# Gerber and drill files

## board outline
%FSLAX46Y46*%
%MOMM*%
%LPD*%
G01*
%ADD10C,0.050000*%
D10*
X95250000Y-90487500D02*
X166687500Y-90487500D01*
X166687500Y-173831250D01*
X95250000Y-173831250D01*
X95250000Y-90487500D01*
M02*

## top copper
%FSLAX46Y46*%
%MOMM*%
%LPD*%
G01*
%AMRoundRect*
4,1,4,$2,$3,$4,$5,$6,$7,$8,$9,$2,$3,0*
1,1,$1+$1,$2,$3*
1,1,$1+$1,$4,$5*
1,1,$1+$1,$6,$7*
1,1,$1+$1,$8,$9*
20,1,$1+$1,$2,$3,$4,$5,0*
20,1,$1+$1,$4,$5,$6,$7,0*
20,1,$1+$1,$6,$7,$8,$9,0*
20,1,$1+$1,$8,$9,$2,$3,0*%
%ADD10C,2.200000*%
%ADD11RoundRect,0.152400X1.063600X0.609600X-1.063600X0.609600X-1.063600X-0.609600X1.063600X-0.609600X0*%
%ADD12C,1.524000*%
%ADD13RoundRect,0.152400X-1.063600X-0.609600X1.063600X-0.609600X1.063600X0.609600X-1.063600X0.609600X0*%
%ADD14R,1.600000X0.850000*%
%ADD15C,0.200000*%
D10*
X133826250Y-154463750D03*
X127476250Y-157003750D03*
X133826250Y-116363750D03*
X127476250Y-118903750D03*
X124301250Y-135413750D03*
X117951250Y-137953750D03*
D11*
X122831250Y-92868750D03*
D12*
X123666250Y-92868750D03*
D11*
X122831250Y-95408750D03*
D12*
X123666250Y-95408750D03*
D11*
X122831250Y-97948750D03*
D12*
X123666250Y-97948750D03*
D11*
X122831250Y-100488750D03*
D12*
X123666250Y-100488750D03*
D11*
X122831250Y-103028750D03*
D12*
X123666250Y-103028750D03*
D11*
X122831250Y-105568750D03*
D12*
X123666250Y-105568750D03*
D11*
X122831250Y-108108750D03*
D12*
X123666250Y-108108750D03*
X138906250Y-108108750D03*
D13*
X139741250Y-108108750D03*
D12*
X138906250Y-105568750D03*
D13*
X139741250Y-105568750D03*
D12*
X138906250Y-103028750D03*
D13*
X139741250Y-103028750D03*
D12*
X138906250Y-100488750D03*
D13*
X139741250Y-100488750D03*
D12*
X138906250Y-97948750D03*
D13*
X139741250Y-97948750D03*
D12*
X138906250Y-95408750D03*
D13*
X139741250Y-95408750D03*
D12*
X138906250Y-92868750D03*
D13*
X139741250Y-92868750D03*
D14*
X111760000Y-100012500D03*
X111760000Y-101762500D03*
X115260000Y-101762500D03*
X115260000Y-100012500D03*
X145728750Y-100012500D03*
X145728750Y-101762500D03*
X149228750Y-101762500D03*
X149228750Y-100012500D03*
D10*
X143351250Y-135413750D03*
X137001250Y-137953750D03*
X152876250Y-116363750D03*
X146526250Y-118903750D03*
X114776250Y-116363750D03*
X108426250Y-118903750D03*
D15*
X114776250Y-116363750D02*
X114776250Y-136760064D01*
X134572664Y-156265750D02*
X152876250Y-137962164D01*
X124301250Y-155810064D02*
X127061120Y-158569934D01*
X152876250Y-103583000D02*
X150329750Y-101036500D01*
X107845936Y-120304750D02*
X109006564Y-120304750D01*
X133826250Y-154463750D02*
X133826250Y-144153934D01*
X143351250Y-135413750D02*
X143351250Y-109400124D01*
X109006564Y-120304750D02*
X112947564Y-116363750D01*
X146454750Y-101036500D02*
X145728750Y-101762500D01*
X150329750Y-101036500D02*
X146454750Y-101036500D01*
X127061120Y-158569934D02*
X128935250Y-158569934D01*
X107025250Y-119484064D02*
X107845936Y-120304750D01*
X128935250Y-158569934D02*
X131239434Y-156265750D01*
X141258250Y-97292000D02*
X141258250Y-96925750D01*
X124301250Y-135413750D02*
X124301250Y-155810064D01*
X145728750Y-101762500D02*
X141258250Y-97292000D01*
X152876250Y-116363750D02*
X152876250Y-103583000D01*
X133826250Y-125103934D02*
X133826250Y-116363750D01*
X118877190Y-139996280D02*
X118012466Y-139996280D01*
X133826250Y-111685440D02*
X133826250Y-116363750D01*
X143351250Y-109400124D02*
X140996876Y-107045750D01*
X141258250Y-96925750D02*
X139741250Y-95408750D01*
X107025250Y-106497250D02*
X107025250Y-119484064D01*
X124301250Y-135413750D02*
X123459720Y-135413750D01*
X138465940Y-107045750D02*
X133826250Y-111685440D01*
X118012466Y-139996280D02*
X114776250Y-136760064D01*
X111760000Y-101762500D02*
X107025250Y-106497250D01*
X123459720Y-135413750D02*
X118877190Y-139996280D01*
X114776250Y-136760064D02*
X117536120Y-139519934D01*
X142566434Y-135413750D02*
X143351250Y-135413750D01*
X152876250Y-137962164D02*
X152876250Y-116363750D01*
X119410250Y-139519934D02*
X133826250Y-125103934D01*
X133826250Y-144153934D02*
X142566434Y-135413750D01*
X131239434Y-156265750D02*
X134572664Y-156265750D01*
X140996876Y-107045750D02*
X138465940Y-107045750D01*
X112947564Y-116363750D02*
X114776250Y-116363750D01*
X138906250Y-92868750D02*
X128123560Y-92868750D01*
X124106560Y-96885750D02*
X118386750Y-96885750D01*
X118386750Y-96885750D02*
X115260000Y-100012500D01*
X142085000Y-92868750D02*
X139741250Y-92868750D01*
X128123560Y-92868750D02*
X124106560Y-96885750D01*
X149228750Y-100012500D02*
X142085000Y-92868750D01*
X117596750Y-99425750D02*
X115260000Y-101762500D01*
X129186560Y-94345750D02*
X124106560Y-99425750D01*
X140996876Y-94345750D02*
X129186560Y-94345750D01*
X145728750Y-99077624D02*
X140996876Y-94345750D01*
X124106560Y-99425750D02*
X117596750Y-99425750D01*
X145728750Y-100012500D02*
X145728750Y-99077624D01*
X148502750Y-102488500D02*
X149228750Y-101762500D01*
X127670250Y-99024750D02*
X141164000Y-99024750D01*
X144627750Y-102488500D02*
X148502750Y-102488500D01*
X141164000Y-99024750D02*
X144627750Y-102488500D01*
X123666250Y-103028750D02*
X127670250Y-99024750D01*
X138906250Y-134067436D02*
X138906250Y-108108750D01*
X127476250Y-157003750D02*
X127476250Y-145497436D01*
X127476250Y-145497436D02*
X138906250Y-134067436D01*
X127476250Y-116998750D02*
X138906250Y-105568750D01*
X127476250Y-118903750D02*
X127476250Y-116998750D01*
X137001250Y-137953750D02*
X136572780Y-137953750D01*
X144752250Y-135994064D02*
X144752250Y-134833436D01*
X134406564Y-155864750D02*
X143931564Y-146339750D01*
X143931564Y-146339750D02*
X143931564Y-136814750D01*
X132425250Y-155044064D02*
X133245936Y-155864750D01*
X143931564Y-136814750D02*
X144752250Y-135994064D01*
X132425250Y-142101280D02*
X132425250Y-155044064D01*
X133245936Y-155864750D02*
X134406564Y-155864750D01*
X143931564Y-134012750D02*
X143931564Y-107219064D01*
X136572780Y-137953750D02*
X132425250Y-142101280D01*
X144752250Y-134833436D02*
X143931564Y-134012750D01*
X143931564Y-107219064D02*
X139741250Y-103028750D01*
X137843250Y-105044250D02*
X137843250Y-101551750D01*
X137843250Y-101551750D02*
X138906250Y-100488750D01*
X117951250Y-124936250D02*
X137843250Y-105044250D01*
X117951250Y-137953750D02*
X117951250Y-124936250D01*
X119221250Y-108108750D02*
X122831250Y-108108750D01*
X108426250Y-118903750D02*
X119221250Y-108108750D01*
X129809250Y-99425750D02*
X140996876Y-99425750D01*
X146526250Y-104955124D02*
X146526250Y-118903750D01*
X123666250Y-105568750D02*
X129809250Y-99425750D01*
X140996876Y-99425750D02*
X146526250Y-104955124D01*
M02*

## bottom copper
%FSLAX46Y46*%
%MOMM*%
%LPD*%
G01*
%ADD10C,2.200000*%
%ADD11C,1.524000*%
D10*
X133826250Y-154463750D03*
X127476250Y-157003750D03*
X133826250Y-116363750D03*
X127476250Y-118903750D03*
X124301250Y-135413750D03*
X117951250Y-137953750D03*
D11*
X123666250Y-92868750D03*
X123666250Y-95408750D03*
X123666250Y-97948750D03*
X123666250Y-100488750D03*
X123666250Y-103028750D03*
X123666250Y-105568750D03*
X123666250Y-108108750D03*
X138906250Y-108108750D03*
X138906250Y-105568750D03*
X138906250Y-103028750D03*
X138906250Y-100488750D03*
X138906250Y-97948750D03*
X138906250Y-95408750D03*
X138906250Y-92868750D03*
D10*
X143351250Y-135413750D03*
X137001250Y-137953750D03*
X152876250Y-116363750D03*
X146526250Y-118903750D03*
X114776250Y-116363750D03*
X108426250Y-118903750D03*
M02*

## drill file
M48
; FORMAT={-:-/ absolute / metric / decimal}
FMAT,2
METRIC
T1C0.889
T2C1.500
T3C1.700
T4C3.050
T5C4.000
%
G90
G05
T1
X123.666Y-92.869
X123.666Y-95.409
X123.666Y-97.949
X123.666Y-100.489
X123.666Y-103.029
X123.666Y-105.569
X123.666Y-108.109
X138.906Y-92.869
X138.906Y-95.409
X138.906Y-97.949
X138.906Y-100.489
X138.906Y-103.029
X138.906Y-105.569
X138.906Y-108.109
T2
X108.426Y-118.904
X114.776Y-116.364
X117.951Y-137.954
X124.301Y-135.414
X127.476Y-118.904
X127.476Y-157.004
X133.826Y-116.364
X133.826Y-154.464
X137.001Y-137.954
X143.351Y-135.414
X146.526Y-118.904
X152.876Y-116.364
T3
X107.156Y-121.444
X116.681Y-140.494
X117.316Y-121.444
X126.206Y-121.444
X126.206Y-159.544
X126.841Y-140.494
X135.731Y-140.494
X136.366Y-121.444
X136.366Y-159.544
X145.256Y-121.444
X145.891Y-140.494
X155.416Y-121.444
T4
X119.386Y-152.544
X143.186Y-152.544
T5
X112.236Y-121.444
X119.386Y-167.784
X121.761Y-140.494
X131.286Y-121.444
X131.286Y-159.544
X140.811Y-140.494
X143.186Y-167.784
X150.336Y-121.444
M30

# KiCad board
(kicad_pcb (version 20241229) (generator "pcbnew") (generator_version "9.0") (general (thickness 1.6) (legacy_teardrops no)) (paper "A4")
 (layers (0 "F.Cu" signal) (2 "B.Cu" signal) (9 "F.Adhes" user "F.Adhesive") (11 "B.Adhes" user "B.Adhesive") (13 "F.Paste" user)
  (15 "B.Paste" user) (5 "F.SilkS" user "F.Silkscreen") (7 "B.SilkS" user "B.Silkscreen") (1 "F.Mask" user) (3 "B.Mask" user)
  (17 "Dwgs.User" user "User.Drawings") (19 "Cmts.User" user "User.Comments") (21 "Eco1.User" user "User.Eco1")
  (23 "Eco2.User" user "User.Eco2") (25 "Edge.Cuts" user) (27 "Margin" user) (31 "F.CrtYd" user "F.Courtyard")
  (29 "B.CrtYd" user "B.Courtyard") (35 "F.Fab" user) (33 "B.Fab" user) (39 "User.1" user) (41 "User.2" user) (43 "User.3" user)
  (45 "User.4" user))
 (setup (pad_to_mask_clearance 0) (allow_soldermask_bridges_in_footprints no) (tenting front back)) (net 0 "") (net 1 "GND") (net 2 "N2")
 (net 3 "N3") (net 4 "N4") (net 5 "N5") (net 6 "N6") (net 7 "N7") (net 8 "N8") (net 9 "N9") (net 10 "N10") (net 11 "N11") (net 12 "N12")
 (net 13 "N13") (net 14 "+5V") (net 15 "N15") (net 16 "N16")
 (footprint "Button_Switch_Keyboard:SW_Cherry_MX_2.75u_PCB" (layer "F.Cu") (at 133.82625 154.46375)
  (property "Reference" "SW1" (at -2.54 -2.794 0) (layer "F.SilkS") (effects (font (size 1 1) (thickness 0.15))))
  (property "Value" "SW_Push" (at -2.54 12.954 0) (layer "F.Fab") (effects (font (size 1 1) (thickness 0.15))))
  (pad "" np_thru_hole circle (at -14.44 -1.92) (size 3.05 3.05) (drill 3.05) (layers "*.Cu" "*.Mask"))
  (pad "" np_thru_hole circle (at -14.44 13.32) (size 4 4) (drill 4) (layers "*.Cu" "*.Mask"))
  (pad "" np_thru_hole circle (at -7.62 5.08) (size 1.7 1.7) (drill 1.7) (layers "*.Cu" "*.Mask"))
  (pad "" np_thru_hole circle (at -2.54 5.08) (size 4 4) (drill 4) (layers "*.Cu" "*.Mask"))
  (pad "" np_thru_hole circle (at 2.54 5.08) (size 1.7 1.7) (drill 1.7) (layers "*.Cu" "*.Mask"))
  (pad "" np_thru_hole circle (at 9.36 -1.92) (size 3.05 3.05) (drill 3.05) (layers "*.Cu" "*.Mask"))
  (pad "" np_thru_hole circle (at 9.36 13.32) (size 4 4) (drill 4) (layers "*.Cu" "*.Mask"))
  (pad "1" thru_hole circle (at 0 0) (size 2.2 2.2) (drill 1.5) (layers "*.Cu" "*.Mask") (remove_unused_layers no) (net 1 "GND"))
  (pad "2" thru_hole circle (at -6.35 2.54) (size 2.2 2.2) (drill 1.5) (layers "*.Cu" "*.Mask") (remove_unused_layers no) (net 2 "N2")))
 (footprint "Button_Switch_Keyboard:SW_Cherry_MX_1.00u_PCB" (layer "F.Cu") (at 133.82625 116.36375)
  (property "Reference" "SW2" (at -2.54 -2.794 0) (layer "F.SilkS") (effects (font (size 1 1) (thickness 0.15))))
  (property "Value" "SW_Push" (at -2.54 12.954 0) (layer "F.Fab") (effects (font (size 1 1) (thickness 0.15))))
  (pad "" np_thru_hole circle (at -7.62 5.08) (size 1.7 1.7) (drill 1.7) (layers "*.Cu" "*.Mask"))
  (pad "" np_thru_hole circle (at -2.54 5.08) (size 4 4) (drill 4) (layers "*.Cu" "*.Mask"))
  (pad "" np_thru_hole circle (at 2.54 5.08) (size 1.7 1.7) (drill 1.7) (layers "*.Cu" "*.Mask"))
  (pad "1" thru_hole circle (at 0 0) (size 2.2 2.2) (drill 1.5) (layers "*.Cu" "*.Mask") (remove_unused_layers no) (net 1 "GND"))
  (pad "2" thru_hole circle (at -6.35 2.54) (size 2.2 2.2) (drill 1.5) (layers "*.Cu" "*.Mask") (remove_unused_layers no) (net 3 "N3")))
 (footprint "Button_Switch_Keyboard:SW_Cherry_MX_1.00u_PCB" (layer "F.Cu") (at 124.30125 135.41375)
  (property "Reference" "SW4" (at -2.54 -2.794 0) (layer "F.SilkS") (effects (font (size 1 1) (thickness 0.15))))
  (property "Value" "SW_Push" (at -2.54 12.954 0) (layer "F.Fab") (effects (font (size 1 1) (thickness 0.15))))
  (pad "" np_thru_hole circle (at -7.62 5.08) (size 1.7 1.7) (drill 1.7) (layers "*.Cu" "*.Mask"))
  (pad "" np_thru_hole circle (at -2.54 5.08) (size 4 4) (drill 4) (layers "*.Cu" "*.Mask"))
  (pad "" np_thru_hole circle (at 2.54 5.08) (size 1.7 1.7) (drill 1.7) (layers "*.Cu" "*.Mask"))
  (pad "1" thru_hole circle (at 0 0) (size 2.2 2.2) (drill 1.5) (layers "*.Cu" "*.Mask") (remove_unused_layers no) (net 1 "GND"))
  (pad "2" thru_hole circle (at -6.35 2.54) (size 2.2 2.2) (drill 1.5) (layers "*.Cu" "*.Mask") (remove_unused_layers no) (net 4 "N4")))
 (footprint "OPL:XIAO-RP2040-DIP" (layer "F.Cu") (at 131.28625 100.48875)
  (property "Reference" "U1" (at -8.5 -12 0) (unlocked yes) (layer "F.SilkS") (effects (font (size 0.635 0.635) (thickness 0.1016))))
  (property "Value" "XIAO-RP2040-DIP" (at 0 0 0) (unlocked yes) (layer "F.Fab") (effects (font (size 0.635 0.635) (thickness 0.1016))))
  (pad "1" smd roundrect (at -8.455 -7.62 180) (size 2.432 1.524) (layers "F.Cu" "F.Mask") (roundrect_rratio 0.1) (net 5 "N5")
   (thermal_bridge_angle 45))
  (pad "1" thru_hole circle (at -7.62 -7.62 180) (size 1.524 1.524) (drill 0.889) (layers "*.Cu" "*.Mask") (remove_unused_layers no)
   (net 5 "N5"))
  (pad "2" smd roundrect (at -8.455 -5.08 180) (size 2.432 1.524) (layers "F.Cu" "F.Mask") (roundrect_rratio 0.1) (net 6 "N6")
   (thermal_bridge_angle 45))
  (pad "2" thru_hole circle (at -7.62 -5.08 180) (size 1.524 1.524) (drill 0.889) (layers "*.Cu" "*.Mask") (remove_unused_layers no)
   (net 6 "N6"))
  (pad "3" smd roundrect (at -8.455 -2.54 180) (size 2.432 1.524) (layers "F.Cu" "F.Mask") (roundrect_rratio 0.1) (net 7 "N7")
   (thermal_bridge_angle 45))
  (pad "3" thru_hole circle (at -7.62 -2.54 180) (size 1.524 1.524) (drill 0.889) (layers "*.Cu" "*.Mask") (remove_unused_layers no)
   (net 7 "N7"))
  (pad "4" smd roundrect (at -8.455 0 180) (size 2.432 1.524) (layers "F.Cu" "F.Mask") (roundrect_rratio 0.1) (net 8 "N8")
   (thermal_bridge_angle 45))
  (pad "4" thru_hole circle (at -7.62 0 180) (size 1.524 1.524) (drill 0.889) (layers "*.Cu" "*.Mask") (remove_unused_layers no)
   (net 8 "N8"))
  (pad "5" smd roundrect (at -8.455 2.54 180) (size 2.432 1.524) (layers "F.Cu" "F.Mask") (roundrect_rratio 0.1) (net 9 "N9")
   (thermal_bridge_angle 45))
  (pad "5" thru_hole circle (at -7.62 2.54 180) (size 1.524 1.524) (drill 0.889) (layers "*.Cu" "*.Mask") (remove_unused_layers no)
   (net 9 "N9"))
  (pad "6" smd roundrect (at -8.455 5.08 180) (size 2.432 1.524) (layers "F.Cu" "F.Mask") (roundrect_rratio 0.1) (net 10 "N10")
   (thermal_bridge_angle 45))
  (pad "6" thru_hole circle (at -7.62 5.08 180) (size 1.524 1.524) (drill 0.889) (layers "*.Cu" "*.Mask") (remove_unused_layers no)
   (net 10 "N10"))
  (pad "7" smd roundrect (at -8.455 7.62 180) (size 2.432 1.524) (layers "F.Cu" "F.Mask") (roundrect_rratio 0.1) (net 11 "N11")
   (thermal_bridge_angle 45))
  (pad "7" thru_hole circle (at -7.62 7.62 180) (size 1.524 1.524) (drill 0.889) (layers "*.Cu" "*.Mask") (remove_unused_layers no)
   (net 11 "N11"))
  (pad "8" thru_hole circle (at 7.62 7.62) (size 1.524 1.524) (drill 0.889) (layers "*.Cu" "*.Mask") (remove_unused_layers no) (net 2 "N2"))
  (pad "8" smd roundrect (at 8.455 7.62) (size 2.432 1.524) (layers "F.Cu" "F.Mask") (roundrect_rratio 0.1) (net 2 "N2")
   (thermal_bridge_angle 45))
  (pad "9" thru_hole circle (at 7.62 5.08) (size 1.524 1.524) (drill 0.889) (layers "*.Cu" "*.Mask") (remove_unused_layers no) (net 3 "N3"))
  (pad "9" smd roundrect (at 8.455 5.08) (size 2.432 1.524) (layers "F.Cu" "F.Mask") (roundrect_rratio 0.1) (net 3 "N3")
   (thermal_bridge_angle 45))
  (pad "10" thru_hole circle (at 7.62 2.54) (size 1.524 1.524) (drill 0.889) (layers "*.Cu" "*.Mask") (remove_unused_layers no)
   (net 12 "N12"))
  (pad "10" smd roundrect (at 8.455 2.54) (size 2.432 1.524) (layers "F.Cu" "F.Mask") (roundrect_rratio 0.1) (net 12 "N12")
   (thermal_bridge_angle 45))
  (pad "11" thru_hole circle (at 7.62 0) (size 1.524 1.524) (drill 0.889) (layers "*.Cu" "*.Mask") (remove_unused_layers no) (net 4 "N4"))
  (pad "11" smd roundrect (at 8.455 0) (size 2.432 1.524) (layers "F.Cu" "F.Mask") (roundrect_rratio 0.1) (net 4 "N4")
   (thermal_bridge_angle 45))
  (pad "12" thru_hole circle (at 7.62 -2.54) (size 1.524 1.524) (drill 0.889) (layers "*.Cu" "*.Mask") (remove_unused_layers no)
   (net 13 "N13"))
  (pad "12" smd roundrect (at 8.455 -2.54) (size 2.432 1.524) (layers "F.Cu" "F.Mask") (roundrect_rratio 0.1) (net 13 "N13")
   (thermal_bridge_angle 45))
  (pad "13" thru_hole circle (at 7.62 -5.08) (size 1.524 1.524) (drill 0.889) (layers "*.Cu" "*.Mask") (remove_unused_layers no)
   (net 1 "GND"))
  (pad "13" smd roundrect (at 8.455 -5.08) (size 2.432 1.524) (layers "F.Cu" "F.Mask") (roundrect_rratio 0.1) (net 1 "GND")
   (thermal_bridge_angle 45))
  (pad "14" thru_hole circle (at 7.62 -7.62) (size 1.524 1.524) (drill 0.889) (layers "*.Cu" "*.Mask") (remove_unused_layers no)
   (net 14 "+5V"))
  (pad "14" smd roundrect (at 8.455 -7.62) (size 2.432 1.524) (layers "F.Cu" "F.Mask") (roundrect_rratio 0.1) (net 14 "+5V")
   (thermal_bridge_angle 45)))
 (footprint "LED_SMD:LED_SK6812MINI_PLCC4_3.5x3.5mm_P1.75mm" (layer "F.Cu") (at 113.51 100.8875)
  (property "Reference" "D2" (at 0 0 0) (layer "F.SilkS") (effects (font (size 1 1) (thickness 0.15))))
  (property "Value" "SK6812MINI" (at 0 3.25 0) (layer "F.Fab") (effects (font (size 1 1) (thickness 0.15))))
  (pad "1" smd rect (at -1.75 -0.875) (size 1.6 0.85) (layers "F.Cu" "F.Mask" "F.Paste") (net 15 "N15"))
  (pad "2" smd rect (at -1.75 0.875) (size 1.6 0.85) (layers "F.Cu" "F.Mask" "F.Paste") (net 1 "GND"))
  (pad "3" smd rect (at 1.75 0.875) (size 1.6 0.85) (layers "F.Cu" "F.Mask" "F.Paste") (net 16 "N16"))
  (pad "4" smd rect (at 1.75 -0.875) (size 1.6 0.85) (layers "F.Cu" "F.Mask" "F.Paste") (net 14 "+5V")))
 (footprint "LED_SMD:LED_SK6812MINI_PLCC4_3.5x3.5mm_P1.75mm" (layer "F.Cu") (at 147.47875 100.8875)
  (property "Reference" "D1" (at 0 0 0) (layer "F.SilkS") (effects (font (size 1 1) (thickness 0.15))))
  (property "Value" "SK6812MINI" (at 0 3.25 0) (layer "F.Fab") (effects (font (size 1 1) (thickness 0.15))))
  (pad "1" smd rect (at -1.75 -0.875) (size 1.6 0.85) (layers "F.Cu" "F.Mask" "F.Paste") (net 16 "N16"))
  (pad "2" smd rect (at -1.75 0.875) (size 1.6 0.85) (layers "F.Cu" "F.Mask" "F.Paste") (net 1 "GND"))
  (pad "3" smd rect (at 1.75 0.875) (size 1.6 0.85) (layers "F.Cu" "F.Mask" "F.Paste") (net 9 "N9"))
  (pad "4" smd rect (at 1.75 -0.875) (size 1.6 0.85) (layers "F.Cu" "F.Mask" "F.Paste") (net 14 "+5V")))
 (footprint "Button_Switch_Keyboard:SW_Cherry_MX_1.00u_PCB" (layer "F.Cu") (at 143.35125 135.41375)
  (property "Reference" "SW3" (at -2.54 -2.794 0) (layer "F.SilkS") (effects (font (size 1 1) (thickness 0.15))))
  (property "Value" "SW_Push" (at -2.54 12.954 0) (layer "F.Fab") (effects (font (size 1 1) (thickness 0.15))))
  (pad "" np_thru_hole circle (at -7.62 5.08) (size 1.7 1.7) (drill 1.7) (layers "*.Cu" "*.Mask"))
  (pad "" np_thru_hole circle (at -2.54 5.08) (size 4 4) (drill 4) (layers "*.Cu" "*.Mask"))
  (pad "" np_thru_hole circle (at 2.54 5.08) (size 1.7 1.7) (drill 1.7) (layers "*.Cu" "*.Mask"))
  (pad "1" thru_hole circle (at 0 0) (size 2.2 2.2) (drill 1.5) (layers "*.Cu" "*.Mask") (remove_unused_layers no) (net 1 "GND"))
  (pad "2" thru_hole circle (at -6.35 2.54) (size 2.2 2.2) (drill 1.5) (layers "*.Cu" "*.Mask") (remove_unused_layers no) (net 12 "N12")))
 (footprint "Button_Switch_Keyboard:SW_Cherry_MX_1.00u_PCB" (layer "F.Cu") (at 152.87625 116.36375)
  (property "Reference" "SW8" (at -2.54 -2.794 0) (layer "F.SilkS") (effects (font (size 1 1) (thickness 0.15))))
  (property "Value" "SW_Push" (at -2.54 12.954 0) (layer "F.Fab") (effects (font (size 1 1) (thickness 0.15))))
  (pad "" np_thru_hole circle (at -7.62 5.08) (size 1.7 1.7) (drill 1.7) (layers "*.Cu" "*.Mask"))
  (pad "" np_thru_hole circle (at -2.54 5.08) (size 4 4) (drill 4) (layers "*.Cu" "*.Mask"))
  (pad "" np_thru_hole circle (at 2.54 5.08) (size 1.7 1.7) (drill 1.7) (layers "*.Cu" "*.Mask"))
  (pad "1" thru_hole circle (at 0 0) (size 2.2 2.2) (drill 1.5) (layers "*.Cu" "*.Mask") (remove_unused_layers no) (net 1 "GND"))
  (pad "2" thru_hole circle (at -6.35 2.54) (size 2.2 2.2) (drill 1.5) (layers "*.Cu" "*.Mask") (remove_unused_layers no) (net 10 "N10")))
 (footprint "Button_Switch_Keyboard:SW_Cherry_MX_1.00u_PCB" (layer "F.Cu") (at 114.77625 116.36375)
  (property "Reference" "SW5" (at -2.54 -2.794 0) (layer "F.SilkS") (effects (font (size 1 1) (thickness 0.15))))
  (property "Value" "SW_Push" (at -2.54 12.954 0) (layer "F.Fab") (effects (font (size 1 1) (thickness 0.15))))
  (pad "" np_thru_hole circle (at -7.62 5.08) (size 1.7 1.7) (drill 1.7) (layers "*.Cu" "*.Mask"))
  (pad "" np_thru_hole circle (at -2.54 5.08) (size 4 4) (drill 4) (layers "*.Cu" "*.Mask"))
  (pad "" np_thru_hole circle (at 2.54 5.08) (size 1.7 1.7) (drill 1.7) (layers "*.Cu" "*.Mask"))
  (pad "1" thru_hole circle (at 0 0) (size 2.2 2.2) (drill 1.5) (layers "*.Cu" "*.Mask") (remove_unused_layers no) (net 1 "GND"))
  (pad "2" thru_hole circle (at -6.35 2.54) (size 2.2 2.2) (drill 1.5) (layers "*.Cu" "*.Mask") (remove_unused_layers no) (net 11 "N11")))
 (gr_rect (start 95.25 90.4875) (end 166.6875 173.83125) (stroke (width 0.05) (type default)) (fill no) (layer "Edge.Cuts"))
 (segment (start 114.77625 116.36375) (end 114.77625 136.760064) (width 0.2) (layer "F.Cu") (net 1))
 (segment (start 134.572664 156.26575) (end 152.87625 137.962164) (width 0.2) (layer "F.Cu") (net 1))
 (segment (start 124.30125 155.810064) (end 127.06112 158.569934) (width 0.2) (layer "F.Cu") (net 1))
 (segment (start 152.87625 103.583) (end 150.32975 101.0365) (width 0.2) (layer "F.Cu") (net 1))
 (segment (start 107.845936 120.30475) (end 109.006564 120.30475) (width 0.2) (layer "F.Cu") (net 1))
 (segment (start 133.82625 154.46375) (end 133.82625 144.153934) (width 0.2) (layer "F.Cu") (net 1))
 (segment (start 143.35125 135.41375) (end 143.35125 109.400124) (width 0.2) (layer "F.Cu") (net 1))
 (segment (start 109.006564 120.30475) (end 112.947564 116.36375) (width 0.2) (layer "F.Cu") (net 1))
 (segment (start 146.45475 101.0365) (end 145.72875 101.7625) (width 0.2) (layer "F.Cu") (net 1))
 (segment (start 150.32975 101.0365) (end 146.45475 101.0365) (width 0.2) (layer "F.Cu") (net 1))
 (segment (start 127.06112 158.569934) (end 128.93525 158.569934) (width 0.2) (layer "F.Cu") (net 1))
 (segment (start 107.02525 119.484064) (end 107.845936 120.30475) (width 0.2) (layer "F.Cu") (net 1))
 (segment (start 128.93525 158.569934) (end 131.239434 156.26575) (width 0.2) (layer "F.Cu") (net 1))
 (segment (start 141.25825 97.292) (end 141.25825 96.92575) (width 0.2) (layer "F.Cu") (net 1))
 (segment (start 124.30125 135.41375) (end 124.30125 155.810064) (width 0.2) (layer "F.Cu") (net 1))
 (segment (start 145.72875 101.7625) (end 141.25825 97.292) (width 0.2) (layer "F.Cu") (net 1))
 (segment (start 152.87625 116.36375) (end 152.87625 103.583) (width 0.2) (layer "F.Cu") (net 1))
 (segment (start 133.82625 125.103934) (end 133.82625 116.36375) (width 0.2) (layer "F.Cu") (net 1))
 (segment (start 118.87719 139.99628) (end 118.012466 139.99628) (width 0.2) (layer "F.Cu") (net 1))
 (segment (start 133.82625 111.68544) (end 133.82625 116.36375) (width 0.2) (layer "F.Cu") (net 1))
 (segment (start 143.35125 109.400124) (end 140.996876 107.04575) (width 0.2) (layer "F.Cu") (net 1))
 (segment (start 141.25825 96.92575) (end 139.74125 95.40875) (width 0.2) (layer "F.Cu") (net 1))
 (segment (start 107.02525 106.49725) (end 107.02525 119.484064) (width 0.2) (layer "F.Cu") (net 1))
 (segment (start 124.30125 135.41375) (end 123.45972 135.41375) (width 0.2) (layer "F.Cu") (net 1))
 (segment (start 138.46594 107.04575) (end 133.82625 111.68544) (width 0.2) (layer "F.Cu") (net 1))
 (segment (start 118.012466 139.99628) (end 114.77625 136.760064) (width 0.2) (layer "F.Cu") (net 1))
 (segment (start 111.76 101.7625) (end 107.02525 106.49725) (width 0.2) (layer "F.Cu") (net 1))
 (segment (start 123.45972 135.41375) (end 118.87719 139.99628) (width 0.2) (layer "F.Cu") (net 1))
 (segment (start 114.77625 136.760064) (end 117.53612 139.519934) (width 0.2) (layer "F.Cu") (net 1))
 (segment (start 142.566434 135.41375) (end 143.35125 135.41375) (width 0.2) (layer "F.Cu") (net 1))
 (segment (start 152.87625 137.962164) (end 152.87625 116.36375) (width 0.2) (layer "F.Cu") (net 1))
 (segment (start 119.41025 139.519934) (end 133.82625 125.103934) (width 0.2) (layer "F.Cu") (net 1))
 (segment (start 133.82625 144.153934) (end 142.566434 135.41375) (width 0.2) (layer "F.Cu") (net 1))
 (segment (start 131.239434 156.26575) (end 134.572664 156.26575) (width 0.2) (layer "F.Cu") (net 1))
 (segment (start 140.996876 107.04575) (end 138.46594 107.04575) (width 0.2) (layer "F.Cu") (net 1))
 (segment (start 112.947564 116.36375) (end 114.77625 116.36375) (width 0.2) (layer "F.Cu") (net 1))
 (segment (start 138.90625 92.86875) (end 128.12356 92.86875) (width 0.2) (layer "F.Cu") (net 14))
 (segment (start 124.10656 96.88575) (end 118.38675 96.88575) (width 0.2) (layer "F.Cu") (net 14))
 (segment (start 118.38675 96.88575) (end 115.26 100.0125) (width 0.2) (layer "F.Cu") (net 14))
 (segment (start 142.085 92.86875) (end 139.74125 92.86875) (width 0.2) (layer "F.Cu") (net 14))
 (segment (start 128.12356 92.86875) (end 124.10656 96.88575) (width 0.2) (layer "F.Cu") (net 14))
 (segment (start 149.22875 100.0125) (end 142.085 92.86875) (width 0.2) (layer "F.Cu") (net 14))
 (segment (start 117.59675 99.42575) (end 115.26 101.7625) (width 0.2) (layer "F.Cu") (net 16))
 (segment (start 129.18656 94.34575) (end 124.10656 99.42575) (width 0.2) (layer "F.Cu") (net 16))
 (segment (start 140.996876 94.34575) (end 129.18656 94.34575) (width 0.2) (layer "F.Cu") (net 16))
 (segment (start 145.72875 99.077624) (end 140.996876 94.34575) (width 0.2) (layer "F.Cu") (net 16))
 (segment (start 124.10656 99.42575) (end 117.59675 99.42575) (width 0.2) (layer "F.Cu") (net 16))
 (segment (start 145.72875 100.0125) (end 145.72875 99.077624) (width 0.2) (layer "F.Cu") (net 16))
 (segment (start 148.50275 102.4885) (end 149.22875 101.7625) (width 0.2) (layer "F.Cu") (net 9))
 (segment (start 127.67025 99.02475) (end 141.164 99.02475) (width 0.2) (layer "F.Cu") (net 9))
 (segment (start 144.62775 102.4885) (end 148.50275 102.4885) (width 0.2) (layer "F.Cu") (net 9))
 (segment (start 141.164 99.02475) (end 144.62775 102.4885) (width 0.2) (layer "F.Cu") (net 9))
 (segment (start 123.66625 103.02875) (end 127.67025 99.02475) (width 0.2) (layer "F.Cu") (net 9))
 (segment (start 138.90625 134.067436) (end 138.90625 108.10875) (width 0.2) (layer "F.Cu") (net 2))
 (segment (start 127.47625 157.00375) (end 127.47625 145.497436) (width 0.2) (layer "F.Cu") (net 2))
 (segment (start 127.47625 145.497436) (end 138.90625 134.067436) (width 0.2) (layer "F.Cu") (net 2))
 (segment (start 127.47625 116.99875) (end 138.90625 105.56875) (width 0.2) (layer "F.Cu") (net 3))
 (segment (start 127.47625 118.90375) (end 127.47625 116.99875) (width 0.2) (layer "F.Cu") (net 3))
 (segment (start 137.00125 137.95375) (end 136.57278 137.95375) (width 0.2) (layer "F.Cu") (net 12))
 (segment (start 144.75225 135.994064) (end 144.75225 134.833436) (width 0.2) (layer "F.Cu") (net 12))
 (segment (start 134.406564 155.86475) (end 143.931564 146.33975) (width 0.2) (layer "F.Cu") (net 12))
 (segment (start 143.931564 146.33975) (end 143.931564 136.81475) (width 0.2) (layer "F.Cu") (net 12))
 (segment (start 132.42525 155.044064) (end 133.245936 155.86475) (width 0.2) (layer "F.Cu") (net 12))
 (segment (start 143.931564 136.81475) (end 144.75225 135.994064) (width 0.2) (layer "F.Cu") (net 12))
 (segment (start 132.42525 142.10128) (end 132.42525 155.044064) (width 0.2) (layer "F.Cu") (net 12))
 (segment (start 133.245936 155.86475) (end 134.406564 155.86475) (width 0.2) (layer "F.Cu") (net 12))
 (segment (start 143.931564 134.01275) (end 143.931564 107.219064) (width 0.2) (layer "F.Cu") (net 12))
 (segment (start 136.57278 137.95375) (end 132.42525 142.10128) (width 0.2) (layer "F.Cu") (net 12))
 (segment (start 144.75225 134.833436) (end 143.931564 134.01275) (width 0.2) (layer "F.Cu") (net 12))
 (segment (start 143.931564 107.219064) (end 139.74125 103.02875) (width 0.2) (layer "F.Cu") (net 12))
 (segment (start 137.84325 105.04425) (end 137.84325 101.55175) (width 0.2) (layer "F.Cu") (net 4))
 (segment (start 137.84325 101.55175) (end 138.90625 100.48875) (width 0.2) (layer "F.Cu") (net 4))
 (segment (start 117.95125 124.93625) (end 137.84325 105.04425) (width 0.2) (layer "F.Cu") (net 4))
 (segment (start 117.95125 137.95375) (end 117.95125 124.93625) (width 0.2) (layer "F.Cu") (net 4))
 (segment (start 119.22125 108.10875) (end 122.83125 108.10875) (width 0.2) (layer "F.Cu") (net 11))
 (segment (start 108.42625 118.90375) (end 119.22125 108.10875) (width 0.2) (layer "F.Cu") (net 11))
 (segment (start 129.80925 99.42575) (end 140.996876 99.42575) (width 0.2) (layer "F.Cu") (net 10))
 (segment (start 146.52625 104.955124) (end 146.52625 118.90375) (width 0.2) (layer "F.Cu") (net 10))
 (segment (start 123.66625 105.56875) (end 129.80925 99.42575) (width 0.2) (layer "F.Cu") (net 10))
 (segment (start 140.996876 99.42575) (end 146.52625 104.955124) (width 0.2) (layer "F.Cu") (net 10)))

